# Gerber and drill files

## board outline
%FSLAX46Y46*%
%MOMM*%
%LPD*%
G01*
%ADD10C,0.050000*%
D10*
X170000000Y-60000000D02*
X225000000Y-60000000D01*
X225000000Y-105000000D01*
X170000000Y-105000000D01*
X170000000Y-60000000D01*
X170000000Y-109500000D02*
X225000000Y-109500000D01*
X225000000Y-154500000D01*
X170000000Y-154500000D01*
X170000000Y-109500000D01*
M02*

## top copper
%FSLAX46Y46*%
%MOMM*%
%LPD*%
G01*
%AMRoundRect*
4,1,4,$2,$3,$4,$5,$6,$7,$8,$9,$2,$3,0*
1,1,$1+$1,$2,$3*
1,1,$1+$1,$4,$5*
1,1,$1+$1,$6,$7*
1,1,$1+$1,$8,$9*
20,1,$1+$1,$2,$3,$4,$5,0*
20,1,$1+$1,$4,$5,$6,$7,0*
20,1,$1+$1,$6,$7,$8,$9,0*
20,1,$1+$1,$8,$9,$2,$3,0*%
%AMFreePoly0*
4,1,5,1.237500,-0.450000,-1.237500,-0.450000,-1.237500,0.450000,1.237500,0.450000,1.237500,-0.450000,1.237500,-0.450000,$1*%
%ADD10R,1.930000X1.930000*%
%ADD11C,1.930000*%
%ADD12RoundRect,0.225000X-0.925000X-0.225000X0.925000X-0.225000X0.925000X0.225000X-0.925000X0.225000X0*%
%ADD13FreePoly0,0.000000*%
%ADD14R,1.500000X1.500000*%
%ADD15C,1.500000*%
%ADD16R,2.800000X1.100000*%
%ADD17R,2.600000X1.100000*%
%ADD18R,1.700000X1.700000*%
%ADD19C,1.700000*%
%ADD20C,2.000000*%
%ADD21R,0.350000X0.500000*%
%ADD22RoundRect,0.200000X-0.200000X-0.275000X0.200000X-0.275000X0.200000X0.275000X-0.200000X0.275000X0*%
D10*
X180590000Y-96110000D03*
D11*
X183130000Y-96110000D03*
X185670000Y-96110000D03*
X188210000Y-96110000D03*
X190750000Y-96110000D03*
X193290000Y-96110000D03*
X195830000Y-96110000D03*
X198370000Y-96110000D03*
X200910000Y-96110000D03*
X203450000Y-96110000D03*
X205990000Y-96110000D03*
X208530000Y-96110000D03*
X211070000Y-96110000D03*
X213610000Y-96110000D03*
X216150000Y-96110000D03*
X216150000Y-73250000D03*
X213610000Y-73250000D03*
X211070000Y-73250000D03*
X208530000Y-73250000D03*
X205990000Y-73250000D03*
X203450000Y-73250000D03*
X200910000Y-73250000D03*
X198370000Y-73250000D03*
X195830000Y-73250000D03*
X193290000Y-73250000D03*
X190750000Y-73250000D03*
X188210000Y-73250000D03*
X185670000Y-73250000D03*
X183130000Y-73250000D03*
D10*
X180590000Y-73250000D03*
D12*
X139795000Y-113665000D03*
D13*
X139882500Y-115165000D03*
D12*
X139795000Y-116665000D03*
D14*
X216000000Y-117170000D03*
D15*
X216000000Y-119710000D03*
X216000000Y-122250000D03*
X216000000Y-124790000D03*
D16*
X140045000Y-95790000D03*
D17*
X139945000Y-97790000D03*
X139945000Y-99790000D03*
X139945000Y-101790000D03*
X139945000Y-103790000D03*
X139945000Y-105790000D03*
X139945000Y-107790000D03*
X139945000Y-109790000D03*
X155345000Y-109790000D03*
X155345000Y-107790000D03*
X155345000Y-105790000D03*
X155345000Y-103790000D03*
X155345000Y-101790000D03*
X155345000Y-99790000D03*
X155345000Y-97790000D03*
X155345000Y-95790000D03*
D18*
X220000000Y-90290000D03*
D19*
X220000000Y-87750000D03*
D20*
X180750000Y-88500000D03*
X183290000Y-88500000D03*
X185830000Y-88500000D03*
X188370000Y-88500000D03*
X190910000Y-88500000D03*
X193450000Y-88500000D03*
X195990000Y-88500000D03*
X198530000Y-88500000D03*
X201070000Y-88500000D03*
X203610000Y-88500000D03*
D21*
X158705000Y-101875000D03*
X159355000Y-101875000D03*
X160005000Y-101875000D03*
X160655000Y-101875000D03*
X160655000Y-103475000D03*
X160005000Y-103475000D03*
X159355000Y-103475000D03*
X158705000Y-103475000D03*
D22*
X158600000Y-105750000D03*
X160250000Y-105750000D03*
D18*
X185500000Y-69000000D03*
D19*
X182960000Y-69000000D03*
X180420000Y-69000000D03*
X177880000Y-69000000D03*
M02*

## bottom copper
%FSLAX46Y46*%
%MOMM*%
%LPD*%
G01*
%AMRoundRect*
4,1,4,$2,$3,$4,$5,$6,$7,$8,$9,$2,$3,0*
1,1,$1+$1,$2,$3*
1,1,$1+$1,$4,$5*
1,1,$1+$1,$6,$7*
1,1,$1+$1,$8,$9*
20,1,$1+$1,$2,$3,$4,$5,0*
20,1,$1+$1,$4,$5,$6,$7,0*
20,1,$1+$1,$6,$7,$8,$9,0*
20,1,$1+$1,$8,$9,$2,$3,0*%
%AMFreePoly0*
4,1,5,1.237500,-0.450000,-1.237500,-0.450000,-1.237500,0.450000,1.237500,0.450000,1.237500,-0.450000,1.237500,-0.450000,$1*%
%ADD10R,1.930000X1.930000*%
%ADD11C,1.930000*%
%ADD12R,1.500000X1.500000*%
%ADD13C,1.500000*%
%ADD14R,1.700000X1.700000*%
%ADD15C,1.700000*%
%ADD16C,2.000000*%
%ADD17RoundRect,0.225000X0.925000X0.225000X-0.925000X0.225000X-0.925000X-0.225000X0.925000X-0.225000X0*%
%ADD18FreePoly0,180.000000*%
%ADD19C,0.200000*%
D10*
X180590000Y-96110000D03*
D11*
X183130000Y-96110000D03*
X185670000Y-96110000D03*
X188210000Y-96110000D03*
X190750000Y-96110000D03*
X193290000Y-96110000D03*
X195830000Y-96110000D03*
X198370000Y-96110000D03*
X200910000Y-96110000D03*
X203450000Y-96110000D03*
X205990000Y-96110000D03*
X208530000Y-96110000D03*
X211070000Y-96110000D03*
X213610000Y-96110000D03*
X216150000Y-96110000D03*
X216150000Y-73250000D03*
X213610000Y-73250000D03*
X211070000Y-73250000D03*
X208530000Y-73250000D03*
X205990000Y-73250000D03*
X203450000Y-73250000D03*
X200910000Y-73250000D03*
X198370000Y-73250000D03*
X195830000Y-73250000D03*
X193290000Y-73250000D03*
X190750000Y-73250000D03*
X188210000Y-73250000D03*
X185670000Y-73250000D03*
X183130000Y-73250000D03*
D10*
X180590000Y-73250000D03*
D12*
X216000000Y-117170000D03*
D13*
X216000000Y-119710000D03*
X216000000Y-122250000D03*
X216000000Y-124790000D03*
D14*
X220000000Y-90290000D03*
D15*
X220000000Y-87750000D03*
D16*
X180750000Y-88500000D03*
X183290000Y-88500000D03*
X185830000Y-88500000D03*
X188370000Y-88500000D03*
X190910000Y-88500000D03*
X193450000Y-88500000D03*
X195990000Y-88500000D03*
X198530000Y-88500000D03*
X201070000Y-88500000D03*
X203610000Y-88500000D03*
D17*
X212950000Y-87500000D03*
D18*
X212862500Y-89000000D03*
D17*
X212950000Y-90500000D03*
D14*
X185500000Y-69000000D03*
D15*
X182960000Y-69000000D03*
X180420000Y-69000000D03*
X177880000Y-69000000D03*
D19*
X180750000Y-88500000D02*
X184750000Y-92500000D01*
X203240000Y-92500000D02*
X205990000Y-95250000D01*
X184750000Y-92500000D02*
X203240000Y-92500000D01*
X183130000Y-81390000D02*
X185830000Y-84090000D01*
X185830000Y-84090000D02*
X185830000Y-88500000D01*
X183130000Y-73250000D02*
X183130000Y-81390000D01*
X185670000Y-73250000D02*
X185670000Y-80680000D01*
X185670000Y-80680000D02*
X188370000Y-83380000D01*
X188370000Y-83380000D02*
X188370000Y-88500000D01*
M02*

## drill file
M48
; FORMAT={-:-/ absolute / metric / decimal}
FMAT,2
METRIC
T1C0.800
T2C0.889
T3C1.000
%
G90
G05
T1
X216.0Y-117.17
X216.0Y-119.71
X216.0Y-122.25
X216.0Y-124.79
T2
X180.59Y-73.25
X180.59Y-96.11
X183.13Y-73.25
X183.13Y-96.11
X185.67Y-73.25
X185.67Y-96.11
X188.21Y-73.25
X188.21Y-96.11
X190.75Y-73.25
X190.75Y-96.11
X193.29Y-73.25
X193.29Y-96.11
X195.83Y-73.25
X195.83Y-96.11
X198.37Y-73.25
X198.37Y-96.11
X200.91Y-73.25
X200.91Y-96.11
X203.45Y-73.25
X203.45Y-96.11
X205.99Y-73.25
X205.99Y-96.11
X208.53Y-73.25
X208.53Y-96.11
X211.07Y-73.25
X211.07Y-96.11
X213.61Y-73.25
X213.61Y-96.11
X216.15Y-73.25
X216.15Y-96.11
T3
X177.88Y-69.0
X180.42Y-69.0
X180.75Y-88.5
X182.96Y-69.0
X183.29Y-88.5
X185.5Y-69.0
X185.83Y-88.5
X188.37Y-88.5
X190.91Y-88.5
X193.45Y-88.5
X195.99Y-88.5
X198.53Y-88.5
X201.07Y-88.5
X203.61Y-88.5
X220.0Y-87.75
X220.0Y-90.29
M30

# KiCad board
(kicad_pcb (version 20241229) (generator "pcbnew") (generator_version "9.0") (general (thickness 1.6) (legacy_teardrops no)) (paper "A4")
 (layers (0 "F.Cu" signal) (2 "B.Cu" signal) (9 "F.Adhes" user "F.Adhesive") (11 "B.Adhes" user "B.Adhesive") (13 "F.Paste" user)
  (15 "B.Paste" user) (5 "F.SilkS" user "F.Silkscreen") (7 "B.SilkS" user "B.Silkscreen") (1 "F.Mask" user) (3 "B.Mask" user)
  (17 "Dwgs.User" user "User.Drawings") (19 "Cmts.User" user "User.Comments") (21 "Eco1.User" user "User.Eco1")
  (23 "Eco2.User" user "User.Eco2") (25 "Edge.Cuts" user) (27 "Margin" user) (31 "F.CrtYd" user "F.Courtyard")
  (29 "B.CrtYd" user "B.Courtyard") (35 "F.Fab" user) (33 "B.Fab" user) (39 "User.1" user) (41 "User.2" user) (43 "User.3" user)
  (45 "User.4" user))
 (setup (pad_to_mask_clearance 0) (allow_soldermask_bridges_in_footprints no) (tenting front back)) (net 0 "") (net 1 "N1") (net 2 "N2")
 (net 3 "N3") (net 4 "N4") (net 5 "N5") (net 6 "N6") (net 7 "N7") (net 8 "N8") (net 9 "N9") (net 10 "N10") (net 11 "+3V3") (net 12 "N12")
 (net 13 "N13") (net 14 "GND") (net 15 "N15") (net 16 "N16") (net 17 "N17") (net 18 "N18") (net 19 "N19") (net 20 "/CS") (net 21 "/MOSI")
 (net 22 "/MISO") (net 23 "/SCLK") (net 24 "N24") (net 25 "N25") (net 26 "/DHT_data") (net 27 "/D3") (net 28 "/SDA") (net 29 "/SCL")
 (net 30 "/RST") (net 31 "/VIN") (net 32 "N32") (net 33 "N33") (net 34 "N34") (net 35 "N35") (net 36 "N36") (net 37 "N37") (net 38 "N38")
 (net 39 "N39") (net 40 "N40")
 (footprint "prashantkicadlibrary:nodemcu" (layer "F.Cu") (at 198.37 84.68 90)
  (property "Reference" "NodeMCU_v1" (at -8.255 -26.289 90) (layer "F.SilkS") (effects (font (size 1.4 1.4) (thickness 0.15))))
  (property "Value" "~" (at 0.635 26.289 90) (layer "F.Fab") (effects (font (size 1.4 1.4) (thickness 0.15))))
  (pad "1" thru_hole rect (at -11.43 -17.78 90) (size 1.93 1.93) (drill 0.889) (layers "*.Cu" "*.Mask") (remove_unused_layers no)
   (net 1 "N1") (solder_mask_margin 0.102))
  (pad "2" thru_hole circle (at -11.43 -15.24 90) (size 1.93 1.93) (drill 0.889) (layers "*.Cu" "*.Mask") (remove_unused_layers no)
   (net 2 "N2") (solder_mask_margin 0.102))
  (pad "3" thru_hole circle (at -11.43 -12.7 90) (size 1.93 1.93) (drill 0.889) (layers "*.Cu" "*.Mask") (remove_unused_layers no)
   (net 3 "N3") (solder_mask_margin 0.102))
  (pad "4" thru_hole circle (at -11.43 -10.16 90) (size 1.93 1.93) (drill 0.889) (layers "*.Cu" "*.Mask") (remove_unused_layers no)
   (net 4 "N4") (solder_mask_margin 0.102))
  (pad "5" thru_hole circle (at -11.43 -7.62 90) (size 1.93 1.93) (drill 0.889) (layers "*.Cu" "*.Mask") (remove_unused_layers no)
   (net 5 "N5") (solder_mask_margin 0.102))
  (pad "6" thru_hole circle (at -11.43 -5.08 90) (size 1.93 1.93) (drill 0.889) (layers "*.Cu" "*.Mask") (remove_unused_layers no)
   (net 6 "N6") (solder_mask_margin 0.102))
  (pad "7" thru_hole circle (at -11.43 -2.54 90) (size 1.93 1.93) (drill 0.889) (layers "*.Cu" "*.Mask") (remove_unused_layers no)
   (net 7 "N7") (solder_mask_margin 0.102))
  (pad "9" thru_hole circle (at -11.43 0 90) (size 1.93 1.93) (drill 0.889) (layers "*.Cu" "*.Mask") (remove_unused_layers no) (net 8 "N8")
   (solder_mask_margin 0.102))
  (pad "9" thru_hole circle (at -11.43 2.54 90) (size 1.93 1.93) (drill 0.889) (layers "*.Cu" "*.Mask") (remove_unused_layers no)
   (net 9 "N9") (solder_mask_margin 0.102))
  (pad "10" thru_hole circle (at -11.43 5.08 90) (size 1.93 1.93) (drill 0.889) (layers "*.Cu" "*.Mask") (remove_unused_layers no)
   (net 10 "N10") (solder_mask_margin 0.102))
  (pad "11" thru_hole circle (at -11.43 7.62 90) (size 1.93 1.93) (drill 0.889) (layers "*.Cu" "*.Mask") (remove_unused_layers no)
   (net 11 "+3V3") (solder_mask_margin 0.102))
  (pad "12" thru_hole circle (at -11.43 10.16 90) (size 1.93 1.93) (drill 0.889) (layers "*.Cu" "*.Mask") (remove_unused_layers no)
   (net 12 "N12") (solder_mask_margin 0.102))
  (pad "13" thru_hole circle (at -11.43 12.7 90) (size 1.93 1.93) (drill 0.889) (layers "*.Cu" "*.Mask") (remove_unused_layers no)
   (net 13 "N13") (solder_mask_margin 0.102))
  (pad "14" thru_hole circle (at -11.43 15.24 90) (size 1.93 1.93) (drill 0.889) (layers "*.Cu" "*.Mask") (remove_unused_layers no)
   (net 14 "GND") (solder_mask_margin 0.102))
  (pad "15" thru_hole circle (at -11.43 17.78 90) (size 1.93 1.93) (drill 0.889) (layers "*.Cu" "*.Mask") (remove_unused_layers no)
   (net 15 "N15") (solder_mask_margin 0.102))
  (pad "16" thru_hole circle (at 11.43 17.78 90) (size 1.93 1.93) (drill 0.889) (layers "*.Cu" "*.Mask") (remove_unused_layers no)
   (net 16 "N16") (solder_mask_margin 0.102))
  (pad "17" thru_hole circle (at 11.43 15.24 90) (size 1.93 1.93) (drill 0.889) (layers "*.Cu" "*.Mask") (remove_unused_layers no)
   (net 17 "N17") (solder_mask_margin 0.102))
  (pad "18" thru_hole circle (at 11.43 12.7 90) (size 1.93 1.93) (drill 0.889) (layers "*.Cu" "*.Mask") (remove_unused_layers no)
   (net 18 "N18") (solder_mask_margin 0.102))
  (pad "19" thru_hole circle (at 11.43 10.16 90) (size 1.93 1.93) (drill 0.889) (layers "*.Cu" "*.Mask") (remove_unused_layers no)
   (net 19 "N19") (solder_mask_margin 0.102))
  (pad "20" thru_hole circle (at 11.43 7.62 90) (size 1.93 1.93) (drill 0.889) (layers "*.Cu" "*.Mask") (remove_unused_layers no)
   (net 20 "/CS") (solder_mask_margin 0.102))
  (pad "21" thru_hole circle (at 11.43 5.08 90) (size 1.93 1.93) (drill 0.889) (layers "*.Cu" "*.Mask") (remove_unused_layers no)
   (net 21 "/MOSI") (solder_mask_margin 0.102))
  (pad "22" thru_hole circle (at 11.43 2.54 90) (size 1.93 1.93) (drill 0.889) (layers "*.Cu" "*.Mask") (remove_unused_layers no)
   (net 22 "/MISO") (solder_mask_margin 0.102))
  (pad "23" thru_hole circle (at 11.43 0 90) (size 1.93 1.93) (drill 0.889) (layers "*.Cu" "*.Mask") (remove_unused_layers no)
   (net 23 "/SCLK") (solder_mask_margin 0.102))
  (pad "24" thru_hole circle (at 11.43 -2.54 90) (size 1.93 1.93) (drill 0.889) (layers "*.Cu" "*.Mask") (remove_unused_layers no)
   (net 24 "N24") (solder_mask_margin 0.102))
  (pad "25" thru_hole circle (at 11.43 -5.08 90) (size 1.93 1.93) (drill 0.889) (layers "*.Cu" "*.Mask") (remove_unused_layers no)
   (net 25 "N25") (solder_mask_margin 0.102))
  (pad "26" thru_hole circle (at 11.43 -7.62 90) (size 1.93 1.93) (drill 0.889) (layers "*.Cu" "*.Mask") (remove_unused_layers no)
   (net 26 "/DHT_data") (solder_mask_margin 0.102))
  (pad "27" thru_hole circle (at 11.43 -10.16 90) (size 1.93 1.93) (drill 0.889) (layers "*.Cu" "*.Mask") (remove_unused_layers no)
   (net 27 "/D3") (solder_mask_margin 0.102))
  (pad "28" thru_hole circle (at 11.43 -12.7 90) (size 1.93 1.93) (drill 0.889) (layers "*.Cu" "*.Mask") (remove_unused_layers no)
   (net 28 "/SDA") (solder_mask_margin 0.102))
  (pad "29" thru_hole circle (at 11.43 -15.24 90) (size 1.93 1.93) (drill 0.889) (layers "*.Cu" "*.Mask") (remove_unused_layers no)
   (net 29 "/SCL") (solder_mask_margin 0.102))
  (pad "30" thru_hole rect (at 11.43 -17.78 90) (size 1.93 1.93) (drill 0.889) (layers "*.Cu" "*.Mask") (remove_unused_layers no)
   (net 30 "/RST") (solder_mask_margin 0.102)))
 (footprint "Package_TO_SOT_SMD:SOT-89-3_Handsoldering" (layer "F.Cu") (at 142.245 115.165)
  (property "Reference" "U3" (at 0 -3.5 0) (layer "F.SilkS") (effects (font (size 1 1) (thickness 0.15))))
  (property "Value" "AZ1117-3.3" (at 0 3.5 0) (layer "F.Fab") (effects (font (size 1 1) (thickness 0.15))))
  (pad "1" smd roundrect (at -2.45 -1.5) (size 2.3 0.9) (layers "F.Cu" "F.Mask" "F.Paste") (roundrect_rratio 0.25) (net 14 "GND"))
  (pad "2" smd custom (at -2.3625 0) (size 2.475 0.9) (layers "F.Cu" "F.Mask" "F.Paste") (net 11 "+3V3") (zone_connect 2)
   (thermal_bridge_angle 45) (options (clearance outline) (anchor rect)) (primitives))
  (pad "3" smd roundrect (at -2.45 1.5) (size 2.3 0.9) (layers "F.Cu" "F.Mask" "F.Paste") (roundrect_rratio 0.25) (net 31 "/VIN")))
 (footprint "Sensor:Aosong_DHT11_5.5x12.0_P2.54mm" (layer "F.Cu") (at 216 117.17)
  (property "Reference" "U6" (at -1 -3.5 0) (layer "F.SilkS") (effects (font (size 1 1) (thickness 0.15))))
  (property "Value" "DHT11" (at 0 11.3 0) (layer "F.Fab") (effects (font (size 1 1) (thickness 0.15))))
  (pad "1" thru_hole rect (at 0 0) (size 1.5 1.5) (drill 0.8) (layers "*.Cu" "*.Mask") (remove_unused_layers no) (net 11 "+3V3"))
  (pad "2" thru_hole circle (at 0 2.54) (size 1.5 1.5) (drill 0.8) (layers "*.Cu" "*.Mask") (remove_unused_layers no) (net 26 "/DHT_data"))
  (pad "3" thru_hole circle (at 0 5.08) (size 1.5 1.5) (drill 0.8) (layers "*.Cu" "*.Mask") (remove_unused_layers no) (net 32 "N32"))
  (pad "4" thru_hole circle (at 0 7.62) (size 1.5 1.5) (drill 0.8) (layers "*.Cu" "*.Mask") (remove_unused_layers no) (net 14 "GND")))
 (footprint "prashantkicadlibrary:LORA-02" (layer "F.Cu") (at 147.645 102.79)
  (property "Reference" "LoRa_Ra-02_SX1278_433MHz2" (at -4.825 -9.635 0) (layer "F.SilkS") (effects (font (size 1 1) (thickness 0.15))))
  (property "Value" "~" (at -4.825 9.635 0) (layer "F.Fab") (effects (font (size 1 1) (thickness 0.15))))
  (pad "1" smd rect (at -7.6 -7) (size 2.8 1.1) (layers "F.Cu" "F.Mask" "F.Paste") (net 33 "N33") (solder_mask_margin 0.102))
  (pad "2" smd rect (at -7.7 -5) (size 2.6 1.1) (layers "F.Cu" "F.Mask" "F.Paste") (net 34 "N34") (solder_mask_margin 0.102))
  (pad "3" smd rect (at -7.7 -3) (size 2.6 1.1) (layers "F.Cu" "F.Mask" "F.Paste") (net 14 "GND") (solder_mask_margin 0.102))
  (pad "4" smd rect (at -7.7 -1) (size 2.6 1.1) (layers "F.Cu" "F.Mask" "F.Paste") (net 20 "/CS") (solder_mask_margin 0.102))
  (pad "5" smd rect (at -7.7 1) (size 2.6 1.1) (layers "F.Cu" "F.Mask" "F.Paste") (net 11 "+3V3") (solder_mask_margin 0.102))
  (pad "6" smd rect (at -7.7 3) (size 2.6 1.1) (layers "F.Cu" "F.Mask" "F.Paste") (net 21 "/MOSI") (solder_mask_margin 0.102))
  (pad "7" smd rect (at -7.7 5) (size 2.6 1.1) (layers "F.Cu" "F.Mask" "F.Paste") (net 27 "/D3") (solder_mask_margin 0.102))
  (pad "8" smd rect (at -7.7 7) (size 2.6 1.1) (layers "F.Cu" "F.Mask" "F.Paste") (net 22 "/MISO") (solder_mask_margin 0.102))
  (pad "9" smd rect (at 7.7 7) (size 2.6 1.1) (layers "F.Cu" "F.Mask" "F.Paste") (solder_mask_margin 0.102))
  (pad "10" smd rect (at 7.7 5) (size 2.6 1.1) (layers "F.Cu" "F.Mask" "F.Paste") (solder_mask_margin 0.102))
  (pad "11" smd rect (at 7.7 3) (size 2.6 1.1) (layers "F.Cu" "F.Mask" "F.Paste") (solder_mask_margin 0.102))
  (pad "12" smd rect (at 7.7 1) (size 2.6 1.1) (layers "F.Cu" "F.Mask" "F.Paste") (solder_mask_margin 0.102))
  (pad "13" smd rect (at 7.7 -1) (size 2.6 1.1) (layers "F.Cu" "F.Mask" "F.Paste") (solder_mask_margin 0.102))
  (pad "14" smd rect (at 7.7 -3) (size 2.6 1.1) (layers "F.Cu" "F.Mask" "F.Paste") (solder_mask_margin 0.102))
  (pad "15" smd rect (at 7.7 -5) (size 2.6 1.1) (layers "F.Cu" "F.Mask" "F.Paste") (solder_mask_margin 0.102))
  (pad "16" smd rect (at 7.7 -7) (size 2.6 1.1) (layers "F.Cu" "F.Mask" "F.Paste") (solder_mask_margin 0.102)))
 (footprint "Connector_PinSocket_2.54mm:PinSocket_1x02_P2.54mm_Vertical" (layer "F.Cu") (at 220 90.29 180)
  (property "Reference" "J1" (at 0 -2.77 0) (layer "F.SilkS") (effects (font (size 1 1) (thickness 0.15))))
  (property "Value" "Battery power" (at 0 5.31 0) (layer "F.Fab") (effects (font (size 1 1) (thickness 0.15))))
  (pad "1" thru_hole rect (at 0 0 180) (size 1.7 1.7) (drill 1) (layers "*.Cu" "*.Mask") (remove_unused_layers no) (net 31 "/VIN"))
  (pad "2" thru_hole circle (at 0 2.54 180) (size 1.7 1.7) (drill 1) (layers "*.Cu" "*.Mask") (remove_unused_layers no) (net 14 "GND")))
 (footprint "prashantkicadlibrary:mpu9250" (layer "F.Cu") (at 193.74 83.5 90)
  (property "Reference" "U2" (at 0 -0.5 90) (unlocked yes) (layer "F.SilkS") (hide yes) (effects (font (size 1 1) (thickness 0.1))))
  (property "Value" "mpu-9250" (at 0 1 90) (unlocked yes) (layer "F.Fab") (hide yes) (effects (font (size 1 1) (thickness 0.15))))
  (pad "1" thru_hole circle (at -5 -12.99 90) (size 2 2) (drill 1) (layers "*.Cu" "*.Mask") (remove_unused_layers no) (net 11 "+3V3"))
  (pad "2" thru_hole circle (at -5 -10.45 90) (size 2 2) (drill 1) (layers "*.Cu" "*.Mask") (remove_unused_layers no) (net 14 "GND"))
  (pad "3" thru_hole circle (at -5 -7.91 90) (size 2 2) (drill 1) (layers "*.Cu" "*.Mask") (remove_unused_layers no) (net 29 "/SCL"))
  (pad "4" thru_hole circle (at -5 -5.37 90) (size 2 2) (drill 1) (layers "*.Cu" "*.Mask") (remove_unused_layers no) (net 28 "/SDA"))
  (pad "5" thru_hole circle (at -5 -2.83 90) (size 2 2) (drill 1) (layers "*.Cu" "*.Mask") (remove_unused_layers no) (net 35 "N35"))
  (pad "6" thru_hole circle (at -5 -0.29 90) (size 2 2) (drill 1) (layers "*.Cu" "*.Mask") (remove_unused_layers no) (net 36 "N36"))
  (pad "7" thru_hole circle (at -5 2.25 90) (size 2 2) (drill 1) (layers "*.Cu" "*.Mask") (remove_unused_layers no) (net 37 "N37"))
  (pad "8" thru_hole circle (at -5 4.79 90) (size 2 2) (drill 1) (layers "*.Cu" "*.Mask") (remove_unused_layers no) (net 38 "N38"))
  (pad "9" thru_hole circle (at -5 7.33 90) (size 2 2) (drill 1) (layers "*.Cu" "*.Mask") (remove_unused_layers no) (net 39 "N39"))
  (pad "10" thru_hole circle (at -5 9.87 90) (size 2 2) (drill 1) (layers "*.Cu" "*.Mask") (remove_unused_layers no) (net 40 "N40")))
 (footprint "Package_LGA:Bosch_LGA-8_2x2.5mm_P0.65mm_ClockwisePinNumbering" (layer "F.Cu") (at 159.68 102.675)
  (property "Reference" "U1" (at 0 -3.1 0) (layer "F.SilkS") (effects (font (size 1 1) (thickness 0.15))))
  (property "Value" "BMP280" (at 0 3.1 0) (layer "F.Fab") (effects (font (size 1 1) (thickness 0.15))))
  (pad "1" smd rect (at -0.975 -0.8 90) (size 0.5 0.35) (layers "F.Cu" "F.Mask" "F.Paste") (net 11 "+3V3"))
  (pad "2" smd rect (at -0.325 -0.8 90) (size 0.5 0.35) (layers "F.Cu" "F.Mask" "F.Paste") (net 14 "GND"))
  (pad "3" smd rect (at 0.325 -0.8 90) (size 0.5 0.35) (layers "F.Cu" "F.Mask" "F.Paste") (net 29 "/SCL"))
  (pad "4" smd rect (at 0.975 -0.8 90) (size 0.5 0.35) (layers "F.Cu" "F.Mask" "F.Paste") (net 28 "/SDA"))
  (pad "5" smd rect (at 0.975 0.8 90) (size 0.5 0.35) (layers "F.Cu" "F.Mask" "F.Paste") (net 11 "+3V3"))
  (pad "6" smd rect (at 0.325 0.8 90) (size 0.5 0.35) (layers "F.Cu" "F.Mask" "F.Paste") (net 14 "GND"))
  (pad "7" smd rect (at -0.325 0.8 90) (size 0.5 0.35) (layers "F.Cu" "F.Mask" "F.Paste"))
  (pad "8" smd rect (at -0.975 0.8 90) (size 0.5 0.35) (layers "F.Cu" "F.Mask" "F.Paste")))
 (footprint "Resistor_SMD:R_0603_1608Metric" (layer "F.Cu") (at 159.425 105.75)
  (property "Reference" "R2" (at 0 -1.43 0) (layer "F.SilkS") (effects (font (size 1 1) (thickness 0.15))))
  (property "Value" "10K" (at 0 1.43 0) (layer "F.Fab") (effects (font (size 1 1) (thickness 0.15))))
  (pad "1" smd roundrect (at -0.825 0) (size 0.8 0.95) (layers "F.Cu" "F.Mask" "F.Paste") (roundrect_rratio 0.25) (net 30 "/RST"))
  (pad "2" smd roundrect (at 0.825 0) (size 0.8 0.95) (layers "F.Cu" "F.Mask" "F.Paste") (roundrect_rratio 0.25) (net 11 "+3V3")))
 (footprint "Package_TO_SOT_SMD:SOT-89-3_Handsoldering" (layer "B.Cu") (at 210.5 89 180)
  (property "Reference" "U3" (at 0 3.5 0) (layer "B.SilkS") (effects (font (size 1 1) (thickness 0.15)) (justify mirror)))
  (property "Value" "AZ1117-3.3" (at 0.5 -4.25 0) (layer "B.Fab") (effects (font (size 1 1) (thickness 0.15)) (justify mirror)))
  (pad "1" smd roundrect (at -2.45 1.5 180) (size 2.3 0.9) (layers "B.Cu" "B.Mask" "B.Paste") (roundrect_rratio 0.25) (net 14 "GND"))
  (pad "2" smd custom (at -2.3625 0 180) (size 2.475 0.9) (layers "B.Cu" "B.Mask" "B.Paste") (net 11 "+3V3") (zone_connect 2)
   (thermal_bridge_angle 45) (options (clearance outline) (anchor rect)) (primitives))
  (pad "3" smd roundrect (at -2.45 -1.5 180) (size 2.3 0.9) (layers "B.Cu" "B.Mask" "B.Paste") (roundrect_rratio 0.25) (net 31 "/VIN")))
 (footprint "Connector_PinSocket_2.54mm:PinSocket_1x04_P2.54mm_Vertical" (layer "B.Cu") (at 185.5 69 90)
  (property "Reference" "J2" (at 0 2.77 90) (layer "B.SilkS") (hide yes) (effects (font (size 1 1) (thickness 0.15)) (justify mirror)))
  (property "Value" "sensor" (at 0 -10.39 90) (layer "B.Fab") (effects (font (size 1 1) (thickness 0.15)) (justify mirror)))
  (pad "1" thru_hole rect (at 0 0 90) (size 1.7 1.7) (drill 1) (layers "*.Cu" "*.Mask") (remove_unused_layers no) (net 14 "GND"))
  (pad "2" thru_hole circle (at 0 -2.54 90) (size 1.7 1.7) (drill 1) (layers "*.Cu" "*.Mask") (remove_unused_layers no) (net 11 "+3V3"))
  (pad "3" thru_hole circle (at 0 -5.08 90) (size 1.7 1.7) (drill 1) (layers "*.Cu" "*.Mask") (remove_unused_layers no) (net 28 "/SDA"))
  (pad "4" thru_hole circle (at 0 -7.62 90) (size 1.7 1.7) (drill 1) (layers "*.Cu" "*.Mask") (remove_unused_layers no) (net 29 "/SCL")))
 (gr_rect (start 170 60) (end 225 105) (stroke (width 0.05) (type solid)) (fill no) (layer "Edge.Cuts"))
 (gr_rect (start 170 109.5) (end 225 154.5) (stroke (width 0.05) (type solid)) (fill no) (layer "Edge.Cuts"))
 (segment (start 180.75 88.5) (end 184.75 92.5) (width 0.2) (layer "B.Cu") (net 11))
 (segment (start 203.24 92.5) (end 205.99 95.25) (width 0.2) (layer "B.Cu") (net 11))
 (segment (start 184.75 92.5) (end 203.24 92.5) (width 0.2) (layer "B.Cu") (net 11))
 (segment (start 183.13 81.39) (end 185.83 84.09) (width 0.2) (layer "B.Cu") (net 29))
 (segment (start 185.83 84.09) (end 185.83 88.5) (width 0.2) (layer "B.Cu") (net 29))
 (segment (start 183.13 73.25) (end 183.13 81.39) (width 0.2) (layer "B.Cu") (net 29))
 (segment (start 185.67 73.25) (end 185.67 80.68) (width 0.2) (layer "B.Cu") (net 28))
 (segment (start 185.67 80.68) (end 188.37 83.38) (width 0.2) (layer "B.Cu") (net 28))
 (segment (start 188.37 83.38) (end 188.37 88.5) (width 0.2) (layer "B.Cu") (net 28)))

